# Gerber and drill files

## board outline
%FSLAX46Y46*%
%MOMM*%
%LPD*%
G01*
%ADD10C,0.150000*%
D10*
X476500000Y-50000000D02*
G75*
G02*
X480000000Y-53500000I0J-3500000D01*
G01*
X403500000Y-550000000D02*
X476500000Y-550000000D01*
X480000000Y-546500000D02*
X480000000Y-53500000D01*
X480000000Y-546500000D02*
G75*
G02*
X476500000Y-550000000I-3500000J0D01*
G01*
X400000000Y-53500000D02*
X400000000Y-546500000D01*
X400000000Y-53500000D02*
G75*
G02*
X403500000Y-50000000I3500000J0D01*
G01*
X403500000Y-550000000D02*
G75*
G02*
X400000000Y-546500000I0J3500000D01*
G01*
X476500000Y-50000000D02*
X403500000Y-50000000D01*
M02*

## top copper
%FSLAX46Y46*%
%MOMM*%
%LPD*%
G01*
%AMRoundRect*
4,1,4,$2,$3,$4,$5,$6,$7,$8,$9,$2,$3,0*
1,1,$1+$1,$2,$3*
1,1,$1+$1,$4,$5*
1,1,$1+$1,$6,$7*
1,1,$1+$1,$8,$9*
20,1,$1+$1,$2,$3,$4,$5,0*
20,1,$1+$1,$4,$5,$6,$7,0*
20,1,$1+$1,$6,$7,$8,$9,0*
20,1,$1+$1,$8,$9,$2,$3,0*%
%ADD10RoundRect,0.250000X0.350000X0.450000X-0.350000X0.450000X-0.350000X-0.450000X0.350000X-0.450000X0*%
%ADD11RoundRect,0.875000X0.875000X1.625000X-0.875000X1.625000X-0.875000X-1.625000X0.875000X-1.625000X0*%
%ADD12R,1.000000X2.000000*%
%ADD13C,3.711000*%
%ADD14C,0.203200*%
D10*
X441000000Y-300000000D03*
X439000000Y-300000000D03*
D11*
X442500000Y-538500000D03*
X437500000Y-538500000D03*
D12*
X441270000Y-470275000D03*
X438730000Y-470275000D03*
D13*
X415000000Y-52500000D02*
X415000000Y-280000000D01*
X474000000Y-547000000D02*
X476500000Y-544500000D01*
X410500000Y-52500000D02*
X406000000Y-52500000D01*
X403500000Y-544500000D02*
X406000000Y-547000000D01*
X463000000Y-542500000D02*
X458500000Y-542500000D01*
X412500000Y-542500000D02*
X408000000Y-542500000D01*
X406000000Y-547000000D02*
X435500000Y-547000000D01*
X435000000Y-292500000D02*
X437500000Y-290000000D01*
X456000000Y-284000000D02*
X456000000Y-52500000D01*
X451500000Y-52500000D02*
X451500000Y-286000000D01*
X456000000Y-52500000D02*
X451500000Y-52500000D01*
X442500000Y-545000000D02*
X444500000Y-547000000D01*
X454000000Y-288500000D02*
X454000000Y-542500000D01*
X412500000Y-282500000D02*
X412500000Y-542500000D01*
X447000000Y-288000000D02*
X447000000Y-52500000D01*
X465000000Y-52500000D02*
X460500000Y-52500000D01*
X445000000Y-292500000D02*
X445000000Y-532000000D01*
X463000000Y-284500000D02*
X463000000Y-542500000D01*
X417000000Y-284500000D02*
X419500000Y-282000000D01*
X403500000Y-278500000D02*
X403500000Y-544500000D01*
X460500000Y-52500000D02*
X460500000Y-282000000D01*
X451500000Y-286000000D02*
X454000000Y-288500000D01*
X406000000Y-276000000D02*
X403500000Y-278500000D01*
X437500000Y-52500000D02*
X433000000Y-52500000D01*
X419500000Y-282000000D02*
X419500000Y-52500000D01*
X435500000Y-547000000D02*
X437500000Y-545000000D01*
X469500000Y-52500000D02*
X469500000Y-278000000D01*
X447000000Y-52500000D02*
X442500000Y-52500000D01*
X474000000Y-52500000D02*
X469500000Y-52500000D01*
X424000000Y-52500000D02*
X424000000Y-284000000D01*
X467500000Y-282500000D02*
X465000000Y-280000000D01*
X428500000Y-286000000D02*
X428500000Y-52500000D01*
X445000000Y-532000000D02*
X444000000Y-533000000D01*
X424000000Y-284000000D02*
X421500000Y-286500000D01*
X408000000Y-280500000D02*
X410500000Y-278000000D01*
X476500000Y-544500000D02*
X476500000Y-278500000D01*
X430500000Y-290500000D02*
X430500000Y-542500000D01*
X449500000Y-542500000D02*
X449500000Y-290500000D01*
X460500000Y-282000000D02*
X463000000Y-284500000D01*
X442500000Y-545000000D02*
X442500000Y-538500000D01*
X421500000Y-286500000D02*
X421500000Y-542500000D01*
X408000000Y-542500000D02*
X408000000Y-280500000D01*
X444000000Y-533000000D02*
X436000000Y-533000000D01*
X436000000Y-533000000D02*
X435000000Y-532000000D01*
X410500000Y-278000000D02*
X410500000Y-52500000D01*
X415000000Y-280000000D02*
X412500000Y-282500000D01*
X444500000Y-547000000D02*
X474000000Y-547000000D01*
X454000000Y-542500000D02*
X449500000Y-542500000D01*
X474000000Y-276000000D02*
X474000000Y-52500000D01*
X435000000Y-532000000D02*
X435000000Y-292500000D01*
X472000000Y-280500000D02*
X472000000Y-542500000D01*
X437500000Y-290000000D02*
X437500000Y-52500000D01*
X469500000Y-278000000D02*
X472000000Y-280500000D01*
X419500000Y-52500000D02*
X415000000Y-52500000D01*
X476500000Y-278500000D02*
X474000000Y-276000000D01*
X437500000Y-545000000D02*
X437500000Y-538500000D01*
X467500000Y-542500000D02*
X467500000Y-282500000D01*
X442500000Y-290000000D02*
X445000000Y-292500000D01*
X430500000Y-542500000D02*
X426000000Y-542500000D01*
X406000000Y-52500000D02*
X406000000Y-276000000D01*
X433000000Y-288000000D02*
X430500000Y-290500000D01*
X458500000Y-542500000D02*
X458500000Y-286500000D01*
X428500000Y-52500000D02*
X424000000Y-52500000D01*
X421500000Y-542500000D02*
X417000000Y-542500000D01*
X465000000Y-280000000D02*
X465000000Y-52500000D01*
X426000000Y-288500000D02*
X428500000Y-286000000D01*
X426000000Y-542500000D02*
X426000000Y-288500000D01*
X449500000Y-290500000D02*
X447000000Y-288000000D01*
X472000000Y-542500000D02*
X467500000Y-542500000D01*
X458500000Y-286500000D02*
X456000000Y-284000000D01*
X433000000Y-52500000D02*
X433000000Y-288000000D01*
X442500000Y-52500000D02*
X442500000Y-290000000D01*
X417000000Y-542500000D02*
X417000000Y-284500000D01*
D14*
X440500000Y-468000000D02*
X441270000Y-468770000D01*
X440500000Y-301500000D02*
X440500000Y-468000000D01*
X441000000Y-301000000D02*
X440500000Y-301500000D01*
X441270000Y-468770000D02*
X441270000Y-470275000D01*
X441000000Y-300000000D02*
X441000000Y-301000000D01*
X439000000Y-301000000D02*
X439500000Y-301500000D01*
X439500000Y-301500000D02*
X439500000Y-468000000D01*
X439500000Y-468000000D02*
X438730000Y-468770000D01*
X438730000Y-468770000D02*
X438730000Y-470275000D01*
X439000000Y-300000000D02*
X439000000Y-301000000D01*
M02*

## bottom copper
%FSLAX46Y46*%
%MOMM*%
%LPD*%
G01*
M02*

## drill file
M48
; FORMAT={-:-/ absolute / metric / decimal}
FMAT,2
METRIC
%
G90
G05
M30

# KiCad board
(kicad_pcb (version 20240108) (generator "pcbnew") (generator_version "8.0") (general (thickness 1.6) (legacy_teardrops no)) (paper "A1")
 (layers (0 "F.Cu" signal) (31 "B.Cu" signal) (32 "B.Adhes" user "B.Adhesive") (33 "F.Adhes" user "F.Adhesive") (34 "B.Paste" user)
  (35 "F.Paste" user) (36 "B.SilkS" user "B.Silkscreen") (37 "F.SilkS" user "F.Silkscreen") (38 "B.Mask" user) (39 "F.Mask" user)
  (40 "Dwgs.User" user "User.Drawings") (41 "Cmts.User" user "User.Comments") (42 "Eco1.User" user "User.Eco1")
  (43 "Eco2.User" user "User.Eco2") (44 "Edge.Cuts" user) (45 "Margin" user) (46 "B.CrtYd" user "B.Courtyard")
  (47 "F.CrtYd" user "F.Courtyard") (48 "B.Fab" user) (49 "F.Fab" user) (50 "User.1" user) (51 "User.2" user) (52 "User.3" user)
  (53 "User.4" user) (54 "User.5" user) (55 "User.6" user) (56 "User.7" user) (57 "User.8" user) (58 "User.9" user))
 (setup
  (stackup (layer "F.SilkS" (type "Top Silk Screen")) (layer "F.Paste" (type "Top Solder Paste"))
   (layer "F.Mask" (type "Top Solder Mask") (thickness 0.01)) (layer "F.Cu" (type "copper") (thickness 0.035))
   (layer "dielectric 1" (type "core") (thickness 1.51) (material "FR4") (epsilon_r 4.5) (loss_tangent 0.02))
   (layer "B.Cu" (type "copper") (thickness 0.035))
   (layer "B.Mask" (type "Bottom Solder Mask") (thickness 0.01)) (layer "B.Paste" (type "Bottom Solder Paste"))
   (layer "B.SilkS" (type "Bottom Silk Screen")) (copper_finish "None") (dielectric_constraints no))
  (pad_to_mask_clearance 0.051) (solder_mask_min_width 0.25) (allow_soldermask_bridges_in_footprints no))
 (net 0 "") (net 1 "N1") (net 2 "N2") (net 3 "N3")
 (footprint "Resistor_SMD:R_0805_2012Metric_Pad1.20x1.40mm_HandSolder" (layer "F.Cu") (at 440 300 180)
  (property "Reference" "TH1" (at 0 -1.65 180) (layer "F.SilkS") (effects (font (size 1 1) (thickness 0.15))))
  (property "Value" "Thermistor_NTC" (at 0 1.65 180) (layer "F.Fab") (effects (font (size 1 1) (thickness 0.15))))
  (pad "1" smd roundrect (at -1 0 180) (size 1.2 1.4) (layers "F.Cu" "F.Paste" "F.Mask") (roundrect_rratio 0.208333) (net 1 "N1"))
  (pad "2" smd roundrect (at 1 0 180) (size 1.2 1.4) (layers "F.Cu" "F.Paste" "F.Mask") (roundrect_rratio 0.208333) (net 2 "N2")))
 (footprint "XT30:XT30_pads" (layer "F.Cu") (at 440 538.5 180)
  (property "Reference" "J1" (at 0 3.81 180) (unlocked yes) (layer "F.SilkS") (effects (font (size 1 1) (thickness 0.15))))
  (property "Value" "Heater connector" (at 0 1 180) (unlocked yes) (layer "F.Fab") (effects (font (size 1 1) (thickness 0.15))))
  (pad "1" smd roundrect (at -2.5 0 180) (size 3.5 5) (layers "F.Cu" "F.Paste" "F.Mask") (roundrect_rratio 0.25) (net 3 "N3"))
  (pad "2" smd roundrect (at 2.5 0 180) (size 3.5 5) (layers "F.Cu" "F.Paste" "F.Mask") (roundrect_rratio 0.25) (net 3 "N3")))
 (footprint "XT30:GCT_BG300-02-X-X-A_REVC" (layer "F.Cu") (at 440 475.5 180)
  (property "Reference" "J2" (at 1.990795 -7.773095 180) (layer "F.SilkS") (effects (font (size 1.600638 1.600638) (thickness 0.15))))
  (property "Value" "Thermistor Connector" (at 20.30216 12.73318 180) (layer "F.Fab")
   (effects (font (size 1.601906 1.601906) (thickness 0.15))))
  (pad "1" smd rect (at -1.27 5.225 180) (size 1 2) (layers "F.Cu" "F.Paste" "F.Mask") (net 1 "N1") (solder_mask_margin 0.102))
  (pad "2" smd rect (at 1.27 5.225 180) (size 1 2) (layers "F.Cu" "F.Paste" "F.Mask") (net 2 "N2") (solder_mask_margin 0.102)))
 (gr_arc (start 476.5 50) (mid 478.974874 51.025126) (end 480 53.5) (stroke (width 0.15) (type default)) (layer "Edge.Cuts"))
 (gr_line (start 403.5 550) (end 476.5 550) (stroke (width 0.15) (type default)) (layer "Edge.Cuts"))
 (gr_line (start 480 546.5) (end 480 53.5) (stroke (width 0.15) (type default)) (layer "Edge.Cuts"))
 (gr_arc (start 480 546.5) (mid 478.974874 548.974874) (end 476.5 550) (stroke (width 0.15) (type default)) (layer "Edge.Cuts"))
 (gr_line (start 400 53.5) (end 400 546.5) (stroke (width 0.15) (type default)) (layer "Edge.Cuts"))
 (gr_arc (start 400 53.5) (mid 401.025126 51.025126) (end 403.5 50) (stroke (width 0.15) (type default)) (layer "Edge.Cuts"))
 (gr_arc (start 403.5 550) (mid 401.025126 548.974874) (end 400 546.5) (stroke (width 0.15) (type default)) (layer "Edge.Cuts"))
 (gr_line (start 476.5 50) (end 403.5 50) (stroke (width 0.15) (type default)) (layer "Edge.Cuts"))
 (segment (start 415 52.5) (end 415 280) (width 3.711) (layer "F.Cu") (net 3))
 (segment (start 474 547) (end 476.5 544.5) (width 3.711) (layer "F.Cu") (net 3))
 (segment (start 410.5 52.5) (end 406 52.5) (width 3.711) (layer "F.Cu") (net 3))
 (segment (start 403.5 544.5) (end 406 547) (width 3.711) (layer "F.Cu") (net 3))
 (segment (start 463 542.5) (end 458.5 542.5) (width 3.711) (layer "F.Cu") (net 3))
 (segment (start 412.5 542.5) (end 408 542.5) (width 3.711) (layer "F.Cu") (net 3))
 (segment (start 406 547) (end 435.5 547) (width 3.711) (layer "F.Cu") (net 3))
 (segment (start 435 292.5) (end 437.5 290) (width 3.711) (layer "F.Cu") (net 3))
 (segment (start 456 284) (end 456 52.5) (width 3.711) (layer "F.Cu") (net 3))
 (segment (start 451.5 52.5) (end 451.5 286) (width 3.711) (layer "F.Cu") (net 3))
 (segment (start 456 52.5) (end 451.5 52.5) (width 3.711) (layer "F.Cu") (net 3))
 (segment (start 442.5 545) (end 444.5 547) (width 3.711) (layer "F.Cu") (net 3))
 (segment (start 454 288.5) (end 454 542.5) (width 3.711) (layer "F.Cu") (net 3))
 (segment (start 412.5 282.5) (end 412.5 542.5) (width 3.711) (layer "F.Cu") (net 3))
 (segment (start 447 288) (end 447 52.5) (width 3.711) (layer "F.Cu") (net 3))
 (segment (start 465 52.5) (end 460.5 52.5) (width 3.711) (layer "F.Cu") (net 3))
 (segment (start 445 292.5) (end 445 532) (width 3.711) (layer "F.Cu") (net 3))
 (segment (start 463 284.5) (end 463 542.5) (width 3.711) (layer "F.Cu") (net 3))
 (segment (start 417 284.5) (end 419.5 282) (width 3.711) (layer "F.Cu") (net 3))
 (segment (start 403.5 278.5) (end 403.5 544.5) (width 3.711) (layer "F.Cu") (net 3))
 (segment (start 460.5 52.5) (end 460.5 282) (width 3.711) (layer "F.Cu") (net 3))
 (segment (start 451.5 286) (end 454 288.5) (width 3.711) (layer "F.Cu") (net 3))
 (segment (start 406 276) (end 403.5 278.5) (width 3.711) (layer "F.Cu") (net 3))
 (segment (start 437.5 52.5) (end 433 52.5) (width 3.711) (layer "F.Cu") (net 3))
 (segment (start 419.5 282) (end 419.5 52.5) (width 3.711) (layer "F.Cu") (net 3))
 (segment (start 435.5 547) (end 437.5 545) (width 3.711) (layer "F.Cu") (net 3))
 (segment (start 469.5 52.5) (end 469.5 278) (width 3.711) (layer "F.Cu") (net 3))
 (segment (start 447 52.5) (end 442.5 52.5) (width 3.711) (layer "F.Cu") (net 3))
 (segment (start 474 52.5) (end 469.5 52.5) (width 3.711) (layer "F.Cu") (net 3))
 (segment (start 424 52.5) (end 424 284) (width 3.711) (layer "F.Cu") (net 3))
 (segment (start 467.5 282.5) (end 465 280) (width 3.711) (layer "F.Cu") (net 3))
 (segment (start 428.5 286) (end 428.5 52.5) (width 3.711) (layer "F.Cu") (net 3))
 (segment (start 445 532) (end 444 533) (width 3.711) (layer "F.Cu") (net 3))
 (segment (start 424 284) (end 421.5 286.5) (width 3.711) (layer "F.Cu") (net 3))
 (segment (start 408 280.5) (end 410.5 278) (width 3.711) (layer "F.Cu") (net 3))
 (segment (start 476.5 544.5) (end 476.5 278.5) (width 3.711) (layer "F.Cu") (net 3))
 (segment (start 430.5 290.5) (end 430.5 542.5) (width 3.711) (layer "F.Cu") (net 3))
 (segment (start 449.5 542.5) (end 449.5 290.5) (width 3.711) (layer "F.Cu") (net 3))
 (segment (start 460.5 282) (end 463 284.5) (width 3.711) (layer "F.Cu") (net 3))
 (segment (start 442.5 545) (end 442.5 538.5) (width 3.711) (layer "F.Cu") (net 3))
 (segment (start 421.5 286.5) (end 421.5 542.5) (width 3.711) (layer "F.Cu") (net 3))
 (segment (start 408 542.5) (end 408 280.5) (width 3.711) (layer "F.Cu") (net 3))
 (segment (start 444 533) (end 436 533) (width 3.711) (layer "F.Cu") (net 3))
 (segment (start 436 533) (end 435 532) (width 3.711) (layer "F.Cu") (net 3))
 (segment (start 410.5 278) (end 410.5 52.5) (width 3.711) (layer "F.Cu") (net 3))
 (segment (start 415 280) (end 412.5 282.5) (width 3.711) (layer "F.Cu") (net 3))
 (segment (start 444.5 547) (end 474 547) (width 3.711) (layer "F.Cu") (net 3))
 (segment (start 454 542.5) (end 449.5 542.5) (width 3.711) (layer "F.Cu") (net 3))
 (segment (start 474 276) (end 474 52.5) (width 3.711) (layer "F.Cu") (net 3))
 (segment (start 435 532) (end 435 292.5) (width 3.711) (layer "F.Cu") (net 3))
 (segment (start 472 280.5) (end 472 542.5) (width 3.711) (layer "F.Cu") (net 3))
 (segment (start 437.5 290) (end 437.5 52.5) (width 3.711) (layer "F.Cu") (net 3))
 (segment (start 469.5 278) (end 472 280.5) (width 3.711) (layer "F.Cu") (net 3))
 (segment (start 419.5 52.5) (end 415 52.5) (width 3.711) (layer "F.Cu") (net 3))
 (segment (start 476.5 278.5) (end 474 276) (width 3.711) (layer "F.Cu") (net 3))
 (segment (start 437.5 545) (end 437.5 538.5) (width 3.711) (layer "F.Cu") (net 3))
 (segment (start 467.5 542.5) (end 467.5 282.5) (width 3.711) (layer "F.Cu") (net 3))
 (segment (start 442.5 290) (end 445 292.5) (width 3.711) (layer "F.Cu") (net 3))
 (segment (start 430.5 542.5) (end 426 542.5) (width 3.711) (layer "F.Cu") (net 3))
 (segment (start 406 52.5) (end 406 276) (width 3.711) (layer "F.Cu") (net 3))
 (segment (start 433 288) (end 430.5 290.5) (width 3.711) (layer "F.Cu") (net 3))
 (segment (start 458.5 542.5) (end 458.5 286.5) (width 3.711) (layer "F.Cu") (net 3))
 (segment (start 428.5 52.5) (end 424 52.5) (width 3.711) (layer "F.Cu") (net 3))
 (segment (start 421.5 542.5) (end 417 542.5) (width 3.711) (layer "F.Cu") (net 3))
 (segment (start 465 280) (end 465 52.5) (width 3.711) (layer "F.Cu") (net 3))
 (segment (start 426 288.5) (end 428.5 286) (width 3.711) (layer "F.Cu") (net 3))
 (segment (start 426 542.5) (end 426 288.5) (width 3.711) (layer "F.Cu") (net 3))
 (segment (start 449.5 290.5) (end 447 288) (width 3.711) (layer "F.Cu") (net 3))
 (segment (start 472 542.5) (end 467.5 542.5) (width 3.711) (layer "F.Cu") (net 3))
 (segment (start 458.5 286.5) (end 456 284) (width 3.711) (layer "F.Cu") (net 3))
 (segment (start 433 52.5) (end 433 288) (width 3.711) (layer "F.Cu") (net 3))
 (segment (start 442.5 52.5) (end 442.5 290) (width 3.711) (layer "F.Cu") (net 3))
 (segment (start 417 542.5) (end 417 284.5) (width 3.711) (layer "F.Cu") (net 3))
 (segment (start 440.5 468) (end 441.27 468.77) (width 0.2032) (layer "F.Cu") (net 1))
 (segment (start 440.5 301.5) (end 440.5 468) (width 0.2032) (layer "F.Cu") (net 1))
 (segment (start 441 301) (end 440.5 301.5) (width 0.2032) (layer "F.Cu") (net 1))
 (segment (start 441.27 468.77) (end 441.27 470.275) (width 0.2032) (layer "F.Cu") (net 1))
 (segment (start 441 300) (end 441 301) (width 0.2032) (layer "F.Cu") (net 1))
 (segment (start 439 301) (end 439.5 301.5) (width 0.2032) (layer "F.Cu") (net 2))
 (segment (start 439.5 301.5) (end 439.5 468) (width 0.2032) (layer "F.Cu") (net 2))
 (segment (start 439.5 468) (end 438.73 468.77) (width 0.2032) (layer "F.Cu") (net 2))
 (segment (start 438.73 468.77) (end 438.73 470.275) (width 0.2032) (layer "F.Cu") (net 2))
 (segment (start 439 300) (end 439 301) (width 0.2032) (layer "F.Cu") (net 2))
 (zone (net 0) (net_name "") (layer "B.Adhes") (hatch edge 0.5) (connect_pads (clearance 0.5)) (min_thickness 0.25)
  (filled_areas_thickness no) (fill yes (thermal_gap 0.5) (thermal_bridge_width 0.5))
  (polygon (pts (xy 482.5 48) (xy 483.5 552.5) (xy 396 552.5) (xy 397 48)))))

